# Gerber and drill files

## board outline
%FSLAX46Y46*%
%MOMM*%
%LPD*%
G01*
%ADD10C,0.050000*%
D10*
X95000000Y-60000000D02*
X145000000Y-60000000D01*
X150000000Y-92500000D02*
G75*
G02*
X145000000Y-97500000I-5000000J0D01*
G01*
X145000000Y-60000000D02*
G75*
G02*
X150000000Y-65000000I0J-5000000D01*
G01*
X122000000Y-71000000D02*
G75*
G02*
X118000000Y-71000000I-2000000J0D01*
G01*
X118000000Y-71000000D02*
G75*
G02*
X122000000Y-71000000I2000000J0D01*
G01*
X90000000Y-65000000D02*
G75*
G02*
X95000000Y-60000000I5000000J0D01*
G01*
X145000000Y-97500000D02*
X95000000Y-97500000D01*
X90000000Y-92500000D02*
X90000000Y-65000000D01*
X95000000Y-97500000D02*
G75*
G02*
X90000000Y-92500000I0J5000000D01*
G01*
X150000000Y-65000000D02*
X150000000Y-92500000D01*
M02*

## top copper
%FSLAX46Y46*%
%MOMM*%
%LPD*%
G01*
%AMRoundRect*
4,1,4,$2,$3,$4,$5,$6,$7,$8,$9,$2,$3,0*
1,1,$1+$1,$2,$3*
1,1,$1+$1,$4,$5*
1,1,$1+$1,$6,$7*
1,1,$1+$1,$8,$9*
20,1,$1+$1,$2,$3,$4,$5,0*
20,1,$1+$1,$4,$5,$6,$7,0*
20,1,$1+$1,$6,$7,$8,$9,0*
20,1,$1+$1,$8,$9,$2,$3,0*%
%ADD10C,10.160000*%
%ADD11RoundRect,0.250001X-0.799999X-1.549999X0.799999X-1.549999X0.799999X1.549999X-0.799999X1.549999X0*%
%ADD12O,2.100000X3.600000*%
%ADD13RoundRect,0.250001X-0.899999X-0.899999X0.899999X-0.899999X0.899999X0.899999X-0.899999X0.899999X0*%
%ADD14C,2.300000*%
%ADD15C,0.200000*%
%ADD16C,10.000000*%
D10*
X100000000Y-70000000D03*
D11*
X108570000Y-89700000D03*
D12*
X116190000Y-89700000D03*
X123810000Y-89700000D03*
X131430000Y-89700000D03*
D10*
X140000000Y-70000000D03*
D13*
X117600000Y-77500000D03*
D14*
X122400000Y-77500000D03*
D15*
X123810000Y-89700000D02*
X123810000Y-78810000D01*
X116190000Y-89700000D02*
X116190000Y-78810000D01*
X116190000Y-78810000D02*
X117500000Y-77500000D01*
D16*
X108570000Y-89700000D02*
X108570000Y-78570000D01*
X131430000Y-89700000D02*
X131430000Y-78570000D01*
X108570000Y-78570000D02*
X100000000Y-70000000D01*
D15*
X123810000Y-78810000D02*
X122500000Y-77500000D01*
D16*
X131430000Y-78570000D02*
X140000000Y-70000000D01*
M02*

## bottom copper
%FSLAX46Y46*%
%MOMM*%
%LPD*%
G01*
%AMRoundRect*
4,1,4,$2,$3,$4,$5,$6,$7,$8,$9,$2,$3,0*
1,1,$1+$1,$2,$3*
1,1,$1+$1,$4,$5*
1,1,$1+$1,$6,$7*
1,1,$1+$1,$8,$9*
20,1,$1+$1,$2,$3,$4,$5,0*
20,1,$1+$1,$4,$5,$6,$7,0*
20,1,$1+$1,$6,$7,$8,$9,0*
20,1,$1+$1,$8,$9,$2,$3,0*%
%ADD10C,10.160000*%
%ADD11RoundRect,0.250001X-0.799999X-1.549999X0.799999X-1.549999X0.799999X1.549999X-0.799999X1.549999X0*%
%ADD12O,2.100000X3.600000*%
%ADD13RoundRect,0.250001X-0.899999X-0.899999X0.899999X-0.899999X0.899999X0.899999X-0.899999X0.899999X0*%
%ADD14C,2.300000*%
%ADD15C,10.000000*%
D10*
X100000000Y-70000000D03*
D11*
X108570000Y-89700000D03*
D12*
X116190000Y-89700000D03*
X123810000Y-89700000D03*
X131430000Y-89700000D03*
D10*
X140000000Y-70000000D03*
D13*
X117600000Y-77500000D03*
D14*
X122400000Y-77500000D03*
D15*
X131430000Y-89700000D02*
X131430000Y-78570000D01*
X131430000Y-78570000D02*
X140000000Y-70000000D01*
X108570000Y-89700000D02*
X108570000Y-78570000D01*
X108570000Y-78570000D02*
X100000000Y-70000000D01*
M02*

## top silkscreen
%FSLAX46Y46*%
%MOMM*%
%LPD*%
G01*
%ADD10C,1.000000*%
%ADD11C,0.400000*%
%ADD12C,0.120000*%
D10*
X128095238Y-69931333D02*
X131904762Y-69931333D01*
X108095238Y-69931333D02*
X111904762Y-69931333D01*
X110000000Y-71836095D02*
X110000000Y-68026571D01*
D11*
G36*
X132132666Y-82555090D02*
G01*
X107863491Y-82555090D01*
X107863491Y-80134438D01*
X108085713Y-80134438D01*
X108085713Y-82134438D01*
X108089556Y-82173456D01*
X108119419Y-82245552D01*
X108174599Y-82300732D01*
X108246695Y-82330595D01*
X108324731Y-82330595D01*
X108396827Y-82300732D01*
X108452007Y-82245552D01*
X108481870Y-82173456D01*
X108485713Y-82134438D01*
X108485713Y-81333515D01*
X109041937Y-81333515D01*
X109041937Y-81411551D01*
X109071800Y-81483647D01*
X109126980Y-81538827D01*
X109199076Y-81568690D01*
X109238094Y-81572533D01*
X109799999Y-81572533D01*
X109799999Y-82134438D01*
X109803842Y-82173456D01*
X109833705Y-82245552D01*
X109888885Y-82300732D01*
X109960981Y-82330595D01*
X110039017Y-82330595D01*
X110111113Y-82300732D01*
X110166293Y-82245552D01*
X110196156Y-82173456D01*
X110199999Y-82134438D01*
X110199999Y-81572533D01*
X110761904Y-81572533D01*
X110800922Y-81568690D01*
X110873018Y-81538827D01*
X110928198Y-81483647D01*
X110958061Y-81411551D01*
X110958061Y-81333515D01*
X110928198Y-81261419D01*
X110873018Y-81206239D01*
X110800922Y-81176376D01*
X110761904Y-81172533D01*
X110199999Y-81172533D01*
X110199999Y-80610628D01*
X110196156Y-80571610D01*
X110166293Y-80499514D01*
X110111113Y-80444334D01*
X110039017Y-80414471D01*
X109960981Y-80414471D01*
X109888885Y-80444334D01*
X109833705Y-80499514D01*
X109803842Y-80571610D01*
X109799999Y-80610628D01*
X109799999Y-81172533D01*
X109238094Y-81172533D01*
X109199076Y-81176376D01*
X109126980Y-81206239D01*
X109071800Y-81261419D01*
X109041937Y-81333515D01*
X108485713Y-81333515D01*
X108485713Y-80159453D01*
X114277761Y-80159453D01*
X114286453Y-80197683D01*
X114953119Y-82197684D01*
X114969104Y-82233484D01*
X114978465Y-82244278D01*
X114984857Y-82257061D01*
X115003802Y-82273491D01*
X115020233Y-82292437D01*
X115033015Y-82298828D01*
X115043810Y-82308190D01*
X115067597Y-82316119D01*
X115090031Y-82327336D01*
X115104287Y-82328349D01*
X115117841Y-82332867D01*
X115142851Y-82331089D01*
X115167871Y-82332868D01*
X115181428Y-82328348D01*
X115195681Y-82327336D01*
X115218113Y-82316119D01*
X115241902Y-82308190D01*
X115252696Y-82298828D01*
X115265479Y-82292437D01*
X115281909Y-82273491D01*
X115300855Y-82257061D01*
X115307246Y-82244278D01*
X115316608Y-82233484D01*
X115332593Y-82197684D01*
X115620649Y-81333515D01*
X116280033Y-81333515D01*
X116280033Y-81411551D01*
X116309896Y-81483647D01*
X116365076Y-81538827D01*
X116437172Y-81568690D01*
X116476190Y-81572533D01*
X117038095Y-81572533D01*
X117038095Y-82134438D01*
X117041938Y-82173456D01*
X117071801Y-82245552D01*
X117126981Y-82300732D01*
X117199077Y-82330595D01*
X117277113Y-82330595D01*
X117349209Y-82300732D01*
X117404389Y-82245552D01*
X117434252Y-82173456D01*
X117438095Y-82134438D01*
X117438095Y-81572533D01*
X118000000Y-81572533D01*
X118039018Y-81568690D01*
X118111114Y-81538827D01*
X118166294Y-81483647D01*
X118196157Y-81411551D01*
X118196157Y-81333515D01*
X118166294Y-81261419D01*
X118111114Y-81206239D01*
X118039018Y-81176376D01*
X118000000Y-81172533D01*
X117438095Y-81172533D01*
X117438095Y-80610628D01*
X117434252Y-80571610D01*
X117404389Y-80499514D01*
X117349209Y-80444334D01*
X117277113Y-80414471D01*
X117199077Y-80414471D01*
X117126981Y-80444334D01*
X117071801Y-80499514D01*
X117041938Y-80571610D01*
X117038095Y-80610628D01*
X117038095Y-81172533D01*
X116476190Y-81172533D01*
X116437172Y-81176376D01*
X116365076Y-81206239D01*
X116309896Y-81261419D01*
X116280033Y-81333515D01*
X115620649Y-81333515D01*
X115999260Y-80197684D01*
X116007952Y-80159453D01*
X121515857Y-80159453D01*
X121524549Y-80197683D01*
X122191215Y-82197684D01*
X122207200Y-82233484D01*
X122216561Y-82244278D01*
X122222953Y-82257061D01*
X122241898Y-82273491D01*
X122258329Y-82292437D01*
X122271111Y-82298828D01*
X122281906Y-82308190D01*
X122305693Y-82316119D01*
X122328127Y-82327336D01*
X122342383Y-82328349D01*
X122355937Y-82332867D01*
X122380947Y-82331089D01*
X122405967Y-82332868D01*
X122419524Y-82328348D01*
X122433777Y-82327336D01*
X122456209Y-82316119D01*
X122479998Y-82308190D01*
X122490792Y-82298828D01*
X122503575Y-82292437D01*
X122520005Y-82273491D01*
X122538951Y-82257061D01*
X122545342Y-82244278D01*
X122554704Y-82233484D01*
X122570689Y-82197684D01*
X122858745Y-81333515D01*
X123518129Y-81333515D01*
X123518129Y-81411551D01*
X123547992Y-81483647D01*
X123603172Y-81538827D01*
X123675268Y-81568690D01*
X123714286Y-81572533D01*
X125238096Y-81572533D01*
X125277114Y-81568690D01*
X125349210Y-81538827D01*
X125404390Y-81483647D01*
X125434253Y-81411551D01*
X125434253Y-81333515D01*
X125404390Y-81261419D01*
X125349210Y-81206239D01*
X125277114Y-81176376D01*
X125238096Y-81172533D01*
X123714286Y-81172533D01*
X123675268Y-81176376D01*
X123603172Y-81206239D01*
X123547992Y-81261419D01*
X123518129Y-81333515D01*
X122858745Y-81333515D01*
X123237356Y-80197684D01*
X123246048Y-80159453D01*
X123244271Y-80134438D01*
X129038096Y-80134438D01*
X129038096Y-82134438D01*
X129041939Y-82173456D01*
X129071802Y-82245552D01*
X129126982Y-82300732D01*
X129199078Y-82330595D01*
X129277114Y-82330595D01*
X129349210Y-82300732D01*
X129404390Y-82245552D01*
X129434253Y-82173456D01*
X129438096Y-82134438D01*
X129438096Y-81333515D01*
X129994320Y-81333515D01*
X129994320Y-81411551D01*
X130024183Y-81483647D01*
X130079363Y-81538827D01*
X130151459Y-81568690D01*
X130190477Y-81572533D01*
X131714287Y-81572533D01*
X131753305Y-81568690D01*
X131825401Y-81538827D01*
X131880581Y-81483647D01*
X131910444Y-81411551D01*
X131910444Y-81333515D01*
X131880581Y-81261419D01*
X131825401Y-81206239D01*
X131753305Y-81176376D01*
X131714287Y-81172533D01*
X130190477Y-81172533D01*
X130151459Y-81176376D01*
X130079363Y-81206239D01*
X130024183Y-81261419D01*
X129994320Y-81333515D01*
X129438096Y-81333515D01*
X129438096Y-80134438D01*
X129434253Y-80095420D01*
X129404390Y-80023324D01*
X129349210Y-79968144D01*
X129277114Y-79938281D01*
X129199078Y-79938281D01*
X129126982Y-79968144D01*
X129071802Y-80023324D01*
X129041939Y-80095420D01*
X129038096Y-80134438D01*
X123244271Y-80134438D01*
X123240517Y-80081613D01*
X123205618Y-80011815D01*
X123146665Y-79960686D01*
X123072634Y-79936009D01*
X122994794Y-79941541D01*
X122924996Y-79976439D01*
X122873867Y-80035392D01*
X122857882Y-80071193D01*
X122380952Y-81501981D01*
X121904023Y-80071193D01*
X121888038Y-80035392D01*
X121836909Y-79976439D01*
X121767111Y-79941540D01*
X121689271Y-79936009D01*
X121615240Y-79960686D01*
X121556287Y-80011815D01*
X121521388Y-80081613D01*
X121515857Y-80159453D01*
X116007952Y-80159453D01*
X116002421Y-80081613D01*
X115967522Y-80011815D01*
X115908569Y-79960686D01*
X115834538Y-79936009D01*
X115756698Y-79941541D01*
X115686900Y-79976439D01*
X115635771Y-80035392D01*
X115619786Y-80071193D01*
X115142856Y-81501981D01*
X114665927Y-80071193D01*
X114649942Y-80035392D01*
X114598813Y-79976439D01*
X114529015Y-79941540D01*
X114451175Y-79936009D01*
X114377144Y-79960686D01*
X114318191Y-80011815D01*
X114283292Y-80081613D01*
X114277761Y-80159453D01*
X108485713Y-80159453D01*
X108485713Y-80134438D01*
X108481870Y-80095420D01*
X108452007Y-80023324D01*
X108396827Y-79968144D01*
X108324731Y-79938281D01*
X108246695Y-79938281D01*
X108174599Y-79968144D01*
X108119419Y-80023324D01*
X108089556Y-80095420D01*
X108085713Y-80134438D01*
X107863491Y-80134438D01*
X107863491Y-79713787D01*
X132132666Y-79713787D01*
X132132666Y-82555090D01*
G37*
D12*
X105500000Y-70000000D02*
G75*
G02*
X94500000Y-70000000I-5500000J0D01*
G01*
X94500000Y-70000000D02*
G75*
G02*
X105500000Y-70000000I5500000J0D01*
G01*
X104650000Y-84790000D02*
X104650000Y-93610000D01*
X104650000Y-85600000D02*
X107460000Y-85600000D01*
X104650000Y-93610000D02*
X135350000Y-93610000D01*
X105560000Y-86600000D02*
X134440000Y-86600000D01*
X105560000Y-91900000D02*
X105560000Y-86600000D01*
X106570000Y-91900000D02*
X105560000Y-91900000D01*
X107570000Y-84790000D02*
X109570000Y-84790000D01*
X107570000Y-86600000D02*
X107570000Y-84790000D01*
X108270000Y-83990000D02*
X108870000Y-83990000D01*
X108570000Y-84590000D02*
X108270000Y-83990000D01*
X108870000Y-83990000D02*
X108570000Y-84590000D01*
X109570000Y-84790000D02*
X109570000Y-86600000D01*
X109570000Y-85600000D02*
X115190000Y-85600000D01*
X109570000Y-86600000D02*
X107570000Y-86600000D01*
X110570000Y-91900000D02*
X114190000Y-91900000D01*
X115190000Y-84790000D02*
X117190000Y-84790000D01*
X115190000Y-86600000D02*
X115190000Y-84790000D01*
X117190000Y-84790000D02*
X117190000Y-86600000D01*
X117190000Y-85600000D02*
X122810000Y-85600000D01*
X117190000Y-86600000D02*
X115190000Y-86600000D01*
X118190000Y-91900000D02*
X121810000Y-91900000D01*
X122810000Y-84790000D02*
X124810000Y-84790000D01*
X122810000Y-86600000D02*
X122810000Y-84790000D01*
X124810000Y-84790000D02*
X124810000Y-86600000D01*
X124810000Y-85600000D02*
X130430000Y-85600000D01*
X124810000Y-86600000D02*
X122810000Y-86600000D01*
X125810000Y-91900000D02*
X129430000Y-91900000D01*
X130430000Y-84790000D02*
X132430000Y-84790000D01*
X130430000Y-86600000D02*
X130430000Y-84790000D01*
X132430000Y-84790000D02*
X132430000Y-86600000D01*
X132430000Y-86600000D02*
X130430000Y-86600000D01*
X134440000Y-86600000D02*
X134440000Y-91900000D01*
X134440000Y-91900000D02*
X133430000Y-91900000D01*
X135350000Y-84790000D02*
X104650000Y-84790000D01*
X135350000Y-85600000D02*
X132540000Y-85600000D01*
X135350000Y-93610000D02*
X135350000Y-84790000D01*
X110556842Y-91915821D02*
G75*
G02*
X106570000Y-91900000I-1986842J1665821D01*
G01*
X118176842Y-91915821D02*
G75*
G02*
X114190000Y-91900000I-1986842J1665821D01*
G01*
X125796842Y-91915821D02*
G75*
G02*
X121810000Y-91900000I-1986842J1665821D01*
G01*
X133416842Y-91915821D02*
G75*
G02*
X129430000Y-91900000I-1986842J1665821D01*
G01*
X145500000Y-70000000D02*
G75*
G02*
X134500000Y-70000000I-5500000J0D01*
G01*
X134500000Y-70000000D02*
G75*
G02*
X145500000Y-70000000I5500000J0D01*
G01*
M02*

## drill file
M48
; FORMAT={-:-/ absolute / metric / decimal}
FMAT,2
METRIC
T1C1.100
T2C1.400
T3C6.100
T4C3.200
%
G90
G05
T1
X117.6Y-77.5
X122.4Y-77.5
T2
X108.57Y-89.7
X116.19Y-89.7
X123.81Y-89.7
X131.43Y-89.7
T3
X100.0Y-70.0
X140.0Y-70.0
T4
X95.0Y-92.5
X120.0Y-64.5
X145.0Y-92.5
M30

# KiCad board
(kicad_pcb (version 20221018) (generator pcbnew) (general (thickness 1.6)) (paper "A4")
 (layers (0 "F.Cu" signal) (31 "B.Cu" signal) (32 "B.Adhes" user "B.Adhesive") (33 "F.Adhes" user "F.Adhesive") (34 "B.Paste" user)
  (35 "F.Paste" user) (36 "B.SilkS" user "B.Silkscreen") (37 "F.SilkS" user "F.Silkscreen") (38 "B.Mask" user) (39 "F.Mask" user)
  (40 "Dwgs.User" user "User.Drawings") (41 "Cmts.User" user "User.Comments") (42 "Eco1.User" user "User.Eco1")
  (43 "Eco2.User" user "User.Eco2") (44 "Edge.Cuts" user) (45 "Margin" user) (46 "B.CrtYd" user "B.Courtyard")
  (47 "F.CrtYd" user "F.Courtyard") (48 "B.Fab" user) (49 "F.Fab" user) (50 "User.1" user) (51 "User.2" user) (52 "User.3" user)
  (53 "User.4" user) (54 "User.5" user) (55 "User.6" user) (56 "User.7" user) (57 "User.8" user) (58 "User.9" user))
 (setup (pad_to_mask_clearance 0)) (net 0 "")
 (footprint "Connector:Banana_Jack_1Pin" (layer "F.Cu") (at 100 70)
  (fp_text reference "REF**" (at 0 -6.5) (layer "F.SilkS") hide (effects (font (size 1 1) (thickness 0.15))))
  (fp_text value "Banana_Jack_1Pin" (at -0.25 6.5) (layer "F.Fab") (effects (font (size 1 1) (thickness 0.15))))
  (fp_circle (center 0 0) (end 5.5 0) (stroke (width 0.12) (type solid)) (fill none) (layer "F.SilkS"))
  (pad "1" thru_hole circle (at 0 0) (size 10.16 10.16) (drill 6.1) (layers "*.Cu" "*.Mask")))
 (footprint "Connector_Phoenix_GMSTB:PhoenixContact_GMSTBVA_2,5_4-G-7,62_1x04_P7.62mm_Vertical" (layer "F.Cu") (at 108.57 89.7)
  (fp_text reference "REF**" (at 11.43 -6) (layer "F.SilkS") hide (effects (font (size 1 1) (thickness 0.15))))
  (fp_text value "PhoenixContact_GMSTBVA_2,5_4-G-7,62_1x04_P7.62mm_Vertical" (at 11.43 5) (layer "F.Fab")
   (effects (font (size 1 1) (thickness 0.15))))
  (fp_line (start -3.92 -4.91) (end -3.92 3.91) (stroke (width 0.12) (type solid)) (layer "F.SilkS"))
  (fp_line (start -3.92 -4.1) (end -1.11 -4.1) (stroke (width 0.12) (type solid)) (layer "F.SilkS"))
  (fp_line (start -3.92 3.91) (end 26.78 3.91) (stroke (width 0.12) (type solid)) (layer "F.SilkS"))
  (fp_line (start -3.01 -3.1) (end 25.87 -3.1) (stroke (width 0.12) (type solid)) (layer "F.SilkS"))
  (fp_line (start -3.01 2.2) (end -3.01 -3.1) (stroke (width 0.12) (type solid)) (layer "F.SilkS"))
  (fp_line (start -2 2.2) (end -3.01 2.2) (stroke (width 0.12) (type solid)) (layer "F.SilkS"))
  (fp_line (start -1 -4.91) (end 1 -4.91) (stroke (width 0.12) (type solid)) (layer "F.SilkS"))
  (fp_line (start -1 -3.1) (end -1 -4.91) (stroke (width 0.12) (type solid)) (layer "F.SilkS"))
  (fp_line (start -0.3 -5.71) (end 0.3 -5.71) (stroke (width 0.12) (type solid)) (layer "F.SilkS"))
  (fp_line (start 0 -5.11) (end -0.3 -5.71) (stroke (width 0.12) (type solid)) (layer "F.SilkS"))
  (fp_line (start 0.3 -5.71) (end 0 -5.11) (stroke (width 0.12) (type solid)) (layer "F.SilkS"))
  (fp_line (start 1 -4.91) (end 1 -3.1) (stroke (width 0.12) (type solid)) (layer "F.SilkS"))
  (fp_line (start 1 -4.1) (end 6.62 -4.1) (stroke (width 0.12) (type solid)) (layer "F.SilkS"))
  (fp_line (start 1 -3.1) (end -1 -3.1) (stroke (width 0.12) (type solid)) (layer "F.SilkS"))
  (fp_line (start 2 2.2) (end 5.62 2.2) (stroke (width 0.12) (type solid)) (layer "F.SilkS"))
  (fp_line (start 6.62 -4.91) (end 8.62 -4.91) (stroke (width 0.12) (type solid)) (layer "F.SilkS"))
  (fp_line (start 6.62 -3.1) (end 6.62 -4.91) (stroke (width 0.12) (type solid)) (layer "F.SilkS"))
  (fp_line (start 8.62 -4.91) (end 8.62 -3.1) (stroke (width 0.12) (type solid)) (layer "F.SilkS"))
  (fp_line (start 8.62 -4.1) (end 14.24 -4.1) (stroke (width 0.12) (type solid)) (layer "F.SilkS"))
  (fp_line (start 8.62 -3.1) (end 6.62 -3.1) (stroke (width 0.12) (type solid)) (layer "F.SilkS"))
  (fp_line (start 9.62 2.2) (end 13.24 2.2) (stroke (width 0.12) (type solid)) (layer "F.SilkS"))
  (fp_line (start 14.24 -4.91) (end 16.24 -4.91) (stroke (width 0.12) (type solid)) (layer "F.SilkS"))
  (fp_line (start 14.24 -3.1) (end 14.24 -4.91) (stroke (width 0.12) (type solid)) (layer "F.SilkS"))
  (fp_line (start 16.24 -4.91) (end 16.24 -3.1) (stroke (width 0.12) (type solid)) (layer "F.SilkS"))
  (fp_line (start 16.24 -4.1) (end 21.86 -4.1) (stroke (width 0.12) (type solid)) (layer "F.SilkS"))
  (fp_line (start 16.24 -3.1) (end 14.24 -3.1) (stroke (width 0.12) (type solid)) (layer "F.SilkS"))
  (fp_line (start 17.24 2.2) (end 20.86 2.2) (stroke (width 0.12) (type solid)) (layer "F.SilkS"))
  (fp_line (start 21.86 -4.91) (end 23.86 -4.91) (stroke (width 0.12) (type solid)) (layer "F.SilkS"))
  (fp_line (start 21.86 -3.1) (end 21.86 -4.91) (stroke (width 0.12) (type solid)) (layer "F.SilkS"))
  (fp_line (start 23.86 -4.91) (end 23.86 -3.1) (stroke (width 0.12) (type solid)) (layer "F.SilkS"))
  (fp_line (start 23.86 -3.1) (end 21.86 -3.1) (stroke (width 0.12) (type solid)) (layer "F.SilkS"))
  (fp_line (start 25.87 -3.1) (end 25.87 2.2) (stroke (width 0.12) (type solid)) (layer "F.SilkS"))
  (fp_line (start 25.87 2.2) (end 24.86 2.2) (stroke (width 0.12) (type solid)) (layer "F.SilkS"))
  (fp_line (start 26.78 -4.91) (end -3.92 -4.91) (stroke (width 0.12) (type solid)) (layer "F.SilkS"))
  (fp_line (start 26.78 -4.1) (end 23.97 -4.1) (stroke (width 0.12) (type solid)) (layer "F.SilkS"))
  (fp_line (start 26.78 3.91) (end 26.78 -4.91) (stroke (width 0.12) (type solid)) (layer "F.SilkS"))
  (fp_arc (start 1.986842 2.215821) (mid -0.010289 3.142758) (end -2 2.2) (stroke (width 0.12) (type solid)) (layer "F.SilkS"))
  (fp_arc (start 9.606842 2.215821) (mid 7.609711 3.142758) (end 5.62 2.2) (stroke (width 0.12) (type solid)) (layer "F.SilkS"))
  (fp_arc (start 17.226842 2.215821) (mid 15.229711 3.142758) (end 13.24 2.2) (stroke (width 0.12) (type solid)) (layer "F.SilkS"))
  (fp_arc (start 24.846842 2.215821) (mid 22.849711 3.142758) (end 20.86 2.2) (stroke (width 0.12) (type solid)) (layer "F.SilkS"))
  (pad "1" thru_hole roundrect (at 0 0) (size 2.1 3.6) (drill 1.5 1.4) (layers "*.Cu" "*.Mask") (roundrect_rratio 0.1190480952))
  (pad "2" thru_hole oval (at 7.62 0) (size 2.1 3.6) (drill 1.5 1.4) (layers "*.Cu" "*.Mask"))
  (pad "3" thru_hole oval (at 15.24 0) (size 2.1 3.6) (drill 1.5 1.4) (layers "*.Cu" "*.Mask"))
  (pad "4" thru_hole oval (at 22.86 0) (size 2.1 3.6) (drill 1.5 1.4) (layers "*.Cu" "*.Mask")))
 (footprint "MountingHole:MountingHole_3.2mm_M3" (layer "F.Cu") (at 145 92.5)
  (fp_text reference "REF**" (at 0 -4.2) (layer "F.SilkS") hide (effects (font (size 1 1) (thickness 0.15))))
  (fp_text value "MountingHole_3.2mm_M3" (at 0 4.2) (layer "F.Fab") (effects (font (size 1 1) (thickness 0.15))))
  (pad "" np_thru_hole circle (at 0 0) (size 3.2 3.2) (drill 3.2) (layers "F&B.Cu" "*.Mask")))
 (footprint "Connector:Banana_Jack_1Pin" (layer "F.Cu") (at 140 70)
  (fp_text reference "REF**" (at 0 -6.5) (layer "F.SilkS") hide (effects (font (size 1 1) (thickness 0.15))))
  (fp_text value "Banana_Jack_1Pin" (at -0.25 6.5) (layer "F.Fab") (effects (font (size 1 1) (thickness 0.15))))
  (fp_circle (center 0 0) (end 5.5 0) (stroke (width 0.12) (type solid)) (fill none) (layer "F.SilkS"))
  (pad "1" thru_hole circle (at 0 0) (size 10.16 10.16) (drill 6.1) (layers "*.Cu" "*.Mask")))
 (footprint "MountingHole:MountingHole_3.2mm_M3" (layer "F.Cu") (at 120 64.5)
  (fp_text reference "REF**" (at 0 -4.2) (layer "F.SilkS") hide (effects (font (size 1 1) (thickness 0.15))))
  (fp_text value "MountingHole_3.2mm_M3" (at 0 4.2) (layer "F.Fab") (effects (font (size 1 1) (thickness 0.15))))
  (pad "" np_thru_hole circle (at 0 0) (size 3.2 3.2) (drill 3.2) (layers "F&B.Cu" "*.Mask")))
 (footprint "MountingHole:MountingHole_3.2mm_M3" (layer "F.Cu") (at 95 92.5)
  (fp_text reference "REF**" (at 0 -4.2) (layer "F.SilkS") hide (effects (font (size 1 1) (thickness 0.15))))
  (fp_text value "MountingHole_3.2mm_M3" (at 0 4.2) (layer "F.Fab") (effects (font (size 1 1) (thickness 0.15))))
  (pad "" np_thru_hole circle (at 0 0) (size 3.2 3.2) (drill 3.2) (layers "*.Cu" "*.Mask")))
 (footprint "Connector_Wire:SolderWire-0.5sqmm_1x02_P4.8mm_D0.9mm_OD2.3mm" (layer "F.Cu") (at 117.6 77.5)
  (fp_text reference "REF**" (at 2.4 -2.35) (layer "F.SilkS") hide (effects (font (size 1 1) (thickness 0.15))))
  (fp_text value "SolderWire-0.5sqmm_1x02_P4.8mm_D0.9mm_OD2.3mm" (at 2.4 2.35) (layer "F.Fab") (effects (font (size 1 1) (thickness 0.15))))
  (pad "1" thru_hole roundrect (at 0 0) (size 2.3 2.3) (drill 1.1) (layers "*.Cu" "*.Mask") (roundrect_rratio 0.108696087))
  (pad "2" thru_hole circle (at 4.8 0) (size 2.3 2.3) (drill 1.1) (layers "*.Cu" "*.Mask")))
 (gr_line (start 95 60) (end 145 60) (stroke (width 0.05) (type default)) (layer "Edge.Cuts"))
 (gr_arc (start 150 92.5) (mid 148.535534 96.035534) (end 145 97.5) (stroke (width 0.05) (type default)) (layer "Edge.Cuts"))
 (gr_arc (start 145 60) (mid 148.535534 61.464466) (end 150 65) (stroke (width 0.05) (type default)) (layer "Edge.Cuts"))
 (gr_circle (center 120 71) (end 122 71) (stroke (width 0.05) (type default)) (fill none) (layer "Edge.Cuts"))
 (gr_arc (start 90 65) (mid 91.464466 61.464466) (end 95 60) (stroke (width 0.05) (type default)) (layer "Edge.Cuts"))
 (gr_line (start 145 97.5) (end 95 97.5) (stroke (width 0.05) (type default)) (layer "Edge.Cuts"))
 (gr_line (start 90 92.5) (end 90 65) (stroke (width 0.05) (type default)) (layer "Edge.Cuts"))
 (gr_arc (start 95 97.5) (mid 91.464466 96.035534) (end 90 92.5) (stroke (width 0.05) (type default)) (layer "Edge.Cuts"))
 (gr_line (start 150 65) (end 150 92.5) (stroke (width 0.05) (type default)) (layer "Edge.Cuts"))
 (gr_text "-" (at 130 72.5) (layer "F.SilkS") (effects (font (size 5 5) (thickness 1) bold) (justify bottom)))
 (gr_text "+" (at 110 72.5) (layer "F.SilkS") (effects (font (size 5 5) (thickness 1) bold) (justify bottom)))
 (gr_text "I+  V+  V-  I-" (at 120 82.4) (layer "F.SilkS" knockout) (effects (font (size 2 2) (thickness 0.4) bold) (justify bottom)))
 (segment (start 123.81 89.7) (end 123.81 78.81) (width 0.2) (layer "F.Cu") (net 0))
 (segment (start 116.19 89.7) (end 116.19 78.81) (width 0.2) (layer "F.Cu") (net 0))
 (segment (start 116.19 78.81) (end 117.5 77.5) (width 0.2) (layer "F.Cu") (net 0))
 (segment (start 108.57 89.7) (end 108.57 78.57) (width 10) (layer "F.Cu") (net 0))
 (segment (start 131.43 89.7) (end 131.43 78.57) (width 10) (layer "F.Cu") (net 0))
 (segment (start 108.57 78.57) (end 100 70) (width 10) (layer "F.Cu") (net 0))
 (segment (start 123.81 78.81) (end 122.5 77.5) (width 0.2) (layer "F.Cu") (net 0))
 (segment (start 131.43 78.57) (end 140 70) (width 10) (layer "F.Cu") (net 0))
 (segment (start 131.43 89.7) (end 131.43 78.57) (width 10) (layer "B.Cu") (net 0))
 (segment (start 131.43 78.57) (end 140 70) (width 10) (layer "B.Cu") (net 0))
 (segment (start 108.57 89.7) (end 108.57 78.57) (width 10) (layer "B.Cu") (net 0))
 (segment (start 108.57 78.57) (end 100 70) (width 10) (layer "B.Cu") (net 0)))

